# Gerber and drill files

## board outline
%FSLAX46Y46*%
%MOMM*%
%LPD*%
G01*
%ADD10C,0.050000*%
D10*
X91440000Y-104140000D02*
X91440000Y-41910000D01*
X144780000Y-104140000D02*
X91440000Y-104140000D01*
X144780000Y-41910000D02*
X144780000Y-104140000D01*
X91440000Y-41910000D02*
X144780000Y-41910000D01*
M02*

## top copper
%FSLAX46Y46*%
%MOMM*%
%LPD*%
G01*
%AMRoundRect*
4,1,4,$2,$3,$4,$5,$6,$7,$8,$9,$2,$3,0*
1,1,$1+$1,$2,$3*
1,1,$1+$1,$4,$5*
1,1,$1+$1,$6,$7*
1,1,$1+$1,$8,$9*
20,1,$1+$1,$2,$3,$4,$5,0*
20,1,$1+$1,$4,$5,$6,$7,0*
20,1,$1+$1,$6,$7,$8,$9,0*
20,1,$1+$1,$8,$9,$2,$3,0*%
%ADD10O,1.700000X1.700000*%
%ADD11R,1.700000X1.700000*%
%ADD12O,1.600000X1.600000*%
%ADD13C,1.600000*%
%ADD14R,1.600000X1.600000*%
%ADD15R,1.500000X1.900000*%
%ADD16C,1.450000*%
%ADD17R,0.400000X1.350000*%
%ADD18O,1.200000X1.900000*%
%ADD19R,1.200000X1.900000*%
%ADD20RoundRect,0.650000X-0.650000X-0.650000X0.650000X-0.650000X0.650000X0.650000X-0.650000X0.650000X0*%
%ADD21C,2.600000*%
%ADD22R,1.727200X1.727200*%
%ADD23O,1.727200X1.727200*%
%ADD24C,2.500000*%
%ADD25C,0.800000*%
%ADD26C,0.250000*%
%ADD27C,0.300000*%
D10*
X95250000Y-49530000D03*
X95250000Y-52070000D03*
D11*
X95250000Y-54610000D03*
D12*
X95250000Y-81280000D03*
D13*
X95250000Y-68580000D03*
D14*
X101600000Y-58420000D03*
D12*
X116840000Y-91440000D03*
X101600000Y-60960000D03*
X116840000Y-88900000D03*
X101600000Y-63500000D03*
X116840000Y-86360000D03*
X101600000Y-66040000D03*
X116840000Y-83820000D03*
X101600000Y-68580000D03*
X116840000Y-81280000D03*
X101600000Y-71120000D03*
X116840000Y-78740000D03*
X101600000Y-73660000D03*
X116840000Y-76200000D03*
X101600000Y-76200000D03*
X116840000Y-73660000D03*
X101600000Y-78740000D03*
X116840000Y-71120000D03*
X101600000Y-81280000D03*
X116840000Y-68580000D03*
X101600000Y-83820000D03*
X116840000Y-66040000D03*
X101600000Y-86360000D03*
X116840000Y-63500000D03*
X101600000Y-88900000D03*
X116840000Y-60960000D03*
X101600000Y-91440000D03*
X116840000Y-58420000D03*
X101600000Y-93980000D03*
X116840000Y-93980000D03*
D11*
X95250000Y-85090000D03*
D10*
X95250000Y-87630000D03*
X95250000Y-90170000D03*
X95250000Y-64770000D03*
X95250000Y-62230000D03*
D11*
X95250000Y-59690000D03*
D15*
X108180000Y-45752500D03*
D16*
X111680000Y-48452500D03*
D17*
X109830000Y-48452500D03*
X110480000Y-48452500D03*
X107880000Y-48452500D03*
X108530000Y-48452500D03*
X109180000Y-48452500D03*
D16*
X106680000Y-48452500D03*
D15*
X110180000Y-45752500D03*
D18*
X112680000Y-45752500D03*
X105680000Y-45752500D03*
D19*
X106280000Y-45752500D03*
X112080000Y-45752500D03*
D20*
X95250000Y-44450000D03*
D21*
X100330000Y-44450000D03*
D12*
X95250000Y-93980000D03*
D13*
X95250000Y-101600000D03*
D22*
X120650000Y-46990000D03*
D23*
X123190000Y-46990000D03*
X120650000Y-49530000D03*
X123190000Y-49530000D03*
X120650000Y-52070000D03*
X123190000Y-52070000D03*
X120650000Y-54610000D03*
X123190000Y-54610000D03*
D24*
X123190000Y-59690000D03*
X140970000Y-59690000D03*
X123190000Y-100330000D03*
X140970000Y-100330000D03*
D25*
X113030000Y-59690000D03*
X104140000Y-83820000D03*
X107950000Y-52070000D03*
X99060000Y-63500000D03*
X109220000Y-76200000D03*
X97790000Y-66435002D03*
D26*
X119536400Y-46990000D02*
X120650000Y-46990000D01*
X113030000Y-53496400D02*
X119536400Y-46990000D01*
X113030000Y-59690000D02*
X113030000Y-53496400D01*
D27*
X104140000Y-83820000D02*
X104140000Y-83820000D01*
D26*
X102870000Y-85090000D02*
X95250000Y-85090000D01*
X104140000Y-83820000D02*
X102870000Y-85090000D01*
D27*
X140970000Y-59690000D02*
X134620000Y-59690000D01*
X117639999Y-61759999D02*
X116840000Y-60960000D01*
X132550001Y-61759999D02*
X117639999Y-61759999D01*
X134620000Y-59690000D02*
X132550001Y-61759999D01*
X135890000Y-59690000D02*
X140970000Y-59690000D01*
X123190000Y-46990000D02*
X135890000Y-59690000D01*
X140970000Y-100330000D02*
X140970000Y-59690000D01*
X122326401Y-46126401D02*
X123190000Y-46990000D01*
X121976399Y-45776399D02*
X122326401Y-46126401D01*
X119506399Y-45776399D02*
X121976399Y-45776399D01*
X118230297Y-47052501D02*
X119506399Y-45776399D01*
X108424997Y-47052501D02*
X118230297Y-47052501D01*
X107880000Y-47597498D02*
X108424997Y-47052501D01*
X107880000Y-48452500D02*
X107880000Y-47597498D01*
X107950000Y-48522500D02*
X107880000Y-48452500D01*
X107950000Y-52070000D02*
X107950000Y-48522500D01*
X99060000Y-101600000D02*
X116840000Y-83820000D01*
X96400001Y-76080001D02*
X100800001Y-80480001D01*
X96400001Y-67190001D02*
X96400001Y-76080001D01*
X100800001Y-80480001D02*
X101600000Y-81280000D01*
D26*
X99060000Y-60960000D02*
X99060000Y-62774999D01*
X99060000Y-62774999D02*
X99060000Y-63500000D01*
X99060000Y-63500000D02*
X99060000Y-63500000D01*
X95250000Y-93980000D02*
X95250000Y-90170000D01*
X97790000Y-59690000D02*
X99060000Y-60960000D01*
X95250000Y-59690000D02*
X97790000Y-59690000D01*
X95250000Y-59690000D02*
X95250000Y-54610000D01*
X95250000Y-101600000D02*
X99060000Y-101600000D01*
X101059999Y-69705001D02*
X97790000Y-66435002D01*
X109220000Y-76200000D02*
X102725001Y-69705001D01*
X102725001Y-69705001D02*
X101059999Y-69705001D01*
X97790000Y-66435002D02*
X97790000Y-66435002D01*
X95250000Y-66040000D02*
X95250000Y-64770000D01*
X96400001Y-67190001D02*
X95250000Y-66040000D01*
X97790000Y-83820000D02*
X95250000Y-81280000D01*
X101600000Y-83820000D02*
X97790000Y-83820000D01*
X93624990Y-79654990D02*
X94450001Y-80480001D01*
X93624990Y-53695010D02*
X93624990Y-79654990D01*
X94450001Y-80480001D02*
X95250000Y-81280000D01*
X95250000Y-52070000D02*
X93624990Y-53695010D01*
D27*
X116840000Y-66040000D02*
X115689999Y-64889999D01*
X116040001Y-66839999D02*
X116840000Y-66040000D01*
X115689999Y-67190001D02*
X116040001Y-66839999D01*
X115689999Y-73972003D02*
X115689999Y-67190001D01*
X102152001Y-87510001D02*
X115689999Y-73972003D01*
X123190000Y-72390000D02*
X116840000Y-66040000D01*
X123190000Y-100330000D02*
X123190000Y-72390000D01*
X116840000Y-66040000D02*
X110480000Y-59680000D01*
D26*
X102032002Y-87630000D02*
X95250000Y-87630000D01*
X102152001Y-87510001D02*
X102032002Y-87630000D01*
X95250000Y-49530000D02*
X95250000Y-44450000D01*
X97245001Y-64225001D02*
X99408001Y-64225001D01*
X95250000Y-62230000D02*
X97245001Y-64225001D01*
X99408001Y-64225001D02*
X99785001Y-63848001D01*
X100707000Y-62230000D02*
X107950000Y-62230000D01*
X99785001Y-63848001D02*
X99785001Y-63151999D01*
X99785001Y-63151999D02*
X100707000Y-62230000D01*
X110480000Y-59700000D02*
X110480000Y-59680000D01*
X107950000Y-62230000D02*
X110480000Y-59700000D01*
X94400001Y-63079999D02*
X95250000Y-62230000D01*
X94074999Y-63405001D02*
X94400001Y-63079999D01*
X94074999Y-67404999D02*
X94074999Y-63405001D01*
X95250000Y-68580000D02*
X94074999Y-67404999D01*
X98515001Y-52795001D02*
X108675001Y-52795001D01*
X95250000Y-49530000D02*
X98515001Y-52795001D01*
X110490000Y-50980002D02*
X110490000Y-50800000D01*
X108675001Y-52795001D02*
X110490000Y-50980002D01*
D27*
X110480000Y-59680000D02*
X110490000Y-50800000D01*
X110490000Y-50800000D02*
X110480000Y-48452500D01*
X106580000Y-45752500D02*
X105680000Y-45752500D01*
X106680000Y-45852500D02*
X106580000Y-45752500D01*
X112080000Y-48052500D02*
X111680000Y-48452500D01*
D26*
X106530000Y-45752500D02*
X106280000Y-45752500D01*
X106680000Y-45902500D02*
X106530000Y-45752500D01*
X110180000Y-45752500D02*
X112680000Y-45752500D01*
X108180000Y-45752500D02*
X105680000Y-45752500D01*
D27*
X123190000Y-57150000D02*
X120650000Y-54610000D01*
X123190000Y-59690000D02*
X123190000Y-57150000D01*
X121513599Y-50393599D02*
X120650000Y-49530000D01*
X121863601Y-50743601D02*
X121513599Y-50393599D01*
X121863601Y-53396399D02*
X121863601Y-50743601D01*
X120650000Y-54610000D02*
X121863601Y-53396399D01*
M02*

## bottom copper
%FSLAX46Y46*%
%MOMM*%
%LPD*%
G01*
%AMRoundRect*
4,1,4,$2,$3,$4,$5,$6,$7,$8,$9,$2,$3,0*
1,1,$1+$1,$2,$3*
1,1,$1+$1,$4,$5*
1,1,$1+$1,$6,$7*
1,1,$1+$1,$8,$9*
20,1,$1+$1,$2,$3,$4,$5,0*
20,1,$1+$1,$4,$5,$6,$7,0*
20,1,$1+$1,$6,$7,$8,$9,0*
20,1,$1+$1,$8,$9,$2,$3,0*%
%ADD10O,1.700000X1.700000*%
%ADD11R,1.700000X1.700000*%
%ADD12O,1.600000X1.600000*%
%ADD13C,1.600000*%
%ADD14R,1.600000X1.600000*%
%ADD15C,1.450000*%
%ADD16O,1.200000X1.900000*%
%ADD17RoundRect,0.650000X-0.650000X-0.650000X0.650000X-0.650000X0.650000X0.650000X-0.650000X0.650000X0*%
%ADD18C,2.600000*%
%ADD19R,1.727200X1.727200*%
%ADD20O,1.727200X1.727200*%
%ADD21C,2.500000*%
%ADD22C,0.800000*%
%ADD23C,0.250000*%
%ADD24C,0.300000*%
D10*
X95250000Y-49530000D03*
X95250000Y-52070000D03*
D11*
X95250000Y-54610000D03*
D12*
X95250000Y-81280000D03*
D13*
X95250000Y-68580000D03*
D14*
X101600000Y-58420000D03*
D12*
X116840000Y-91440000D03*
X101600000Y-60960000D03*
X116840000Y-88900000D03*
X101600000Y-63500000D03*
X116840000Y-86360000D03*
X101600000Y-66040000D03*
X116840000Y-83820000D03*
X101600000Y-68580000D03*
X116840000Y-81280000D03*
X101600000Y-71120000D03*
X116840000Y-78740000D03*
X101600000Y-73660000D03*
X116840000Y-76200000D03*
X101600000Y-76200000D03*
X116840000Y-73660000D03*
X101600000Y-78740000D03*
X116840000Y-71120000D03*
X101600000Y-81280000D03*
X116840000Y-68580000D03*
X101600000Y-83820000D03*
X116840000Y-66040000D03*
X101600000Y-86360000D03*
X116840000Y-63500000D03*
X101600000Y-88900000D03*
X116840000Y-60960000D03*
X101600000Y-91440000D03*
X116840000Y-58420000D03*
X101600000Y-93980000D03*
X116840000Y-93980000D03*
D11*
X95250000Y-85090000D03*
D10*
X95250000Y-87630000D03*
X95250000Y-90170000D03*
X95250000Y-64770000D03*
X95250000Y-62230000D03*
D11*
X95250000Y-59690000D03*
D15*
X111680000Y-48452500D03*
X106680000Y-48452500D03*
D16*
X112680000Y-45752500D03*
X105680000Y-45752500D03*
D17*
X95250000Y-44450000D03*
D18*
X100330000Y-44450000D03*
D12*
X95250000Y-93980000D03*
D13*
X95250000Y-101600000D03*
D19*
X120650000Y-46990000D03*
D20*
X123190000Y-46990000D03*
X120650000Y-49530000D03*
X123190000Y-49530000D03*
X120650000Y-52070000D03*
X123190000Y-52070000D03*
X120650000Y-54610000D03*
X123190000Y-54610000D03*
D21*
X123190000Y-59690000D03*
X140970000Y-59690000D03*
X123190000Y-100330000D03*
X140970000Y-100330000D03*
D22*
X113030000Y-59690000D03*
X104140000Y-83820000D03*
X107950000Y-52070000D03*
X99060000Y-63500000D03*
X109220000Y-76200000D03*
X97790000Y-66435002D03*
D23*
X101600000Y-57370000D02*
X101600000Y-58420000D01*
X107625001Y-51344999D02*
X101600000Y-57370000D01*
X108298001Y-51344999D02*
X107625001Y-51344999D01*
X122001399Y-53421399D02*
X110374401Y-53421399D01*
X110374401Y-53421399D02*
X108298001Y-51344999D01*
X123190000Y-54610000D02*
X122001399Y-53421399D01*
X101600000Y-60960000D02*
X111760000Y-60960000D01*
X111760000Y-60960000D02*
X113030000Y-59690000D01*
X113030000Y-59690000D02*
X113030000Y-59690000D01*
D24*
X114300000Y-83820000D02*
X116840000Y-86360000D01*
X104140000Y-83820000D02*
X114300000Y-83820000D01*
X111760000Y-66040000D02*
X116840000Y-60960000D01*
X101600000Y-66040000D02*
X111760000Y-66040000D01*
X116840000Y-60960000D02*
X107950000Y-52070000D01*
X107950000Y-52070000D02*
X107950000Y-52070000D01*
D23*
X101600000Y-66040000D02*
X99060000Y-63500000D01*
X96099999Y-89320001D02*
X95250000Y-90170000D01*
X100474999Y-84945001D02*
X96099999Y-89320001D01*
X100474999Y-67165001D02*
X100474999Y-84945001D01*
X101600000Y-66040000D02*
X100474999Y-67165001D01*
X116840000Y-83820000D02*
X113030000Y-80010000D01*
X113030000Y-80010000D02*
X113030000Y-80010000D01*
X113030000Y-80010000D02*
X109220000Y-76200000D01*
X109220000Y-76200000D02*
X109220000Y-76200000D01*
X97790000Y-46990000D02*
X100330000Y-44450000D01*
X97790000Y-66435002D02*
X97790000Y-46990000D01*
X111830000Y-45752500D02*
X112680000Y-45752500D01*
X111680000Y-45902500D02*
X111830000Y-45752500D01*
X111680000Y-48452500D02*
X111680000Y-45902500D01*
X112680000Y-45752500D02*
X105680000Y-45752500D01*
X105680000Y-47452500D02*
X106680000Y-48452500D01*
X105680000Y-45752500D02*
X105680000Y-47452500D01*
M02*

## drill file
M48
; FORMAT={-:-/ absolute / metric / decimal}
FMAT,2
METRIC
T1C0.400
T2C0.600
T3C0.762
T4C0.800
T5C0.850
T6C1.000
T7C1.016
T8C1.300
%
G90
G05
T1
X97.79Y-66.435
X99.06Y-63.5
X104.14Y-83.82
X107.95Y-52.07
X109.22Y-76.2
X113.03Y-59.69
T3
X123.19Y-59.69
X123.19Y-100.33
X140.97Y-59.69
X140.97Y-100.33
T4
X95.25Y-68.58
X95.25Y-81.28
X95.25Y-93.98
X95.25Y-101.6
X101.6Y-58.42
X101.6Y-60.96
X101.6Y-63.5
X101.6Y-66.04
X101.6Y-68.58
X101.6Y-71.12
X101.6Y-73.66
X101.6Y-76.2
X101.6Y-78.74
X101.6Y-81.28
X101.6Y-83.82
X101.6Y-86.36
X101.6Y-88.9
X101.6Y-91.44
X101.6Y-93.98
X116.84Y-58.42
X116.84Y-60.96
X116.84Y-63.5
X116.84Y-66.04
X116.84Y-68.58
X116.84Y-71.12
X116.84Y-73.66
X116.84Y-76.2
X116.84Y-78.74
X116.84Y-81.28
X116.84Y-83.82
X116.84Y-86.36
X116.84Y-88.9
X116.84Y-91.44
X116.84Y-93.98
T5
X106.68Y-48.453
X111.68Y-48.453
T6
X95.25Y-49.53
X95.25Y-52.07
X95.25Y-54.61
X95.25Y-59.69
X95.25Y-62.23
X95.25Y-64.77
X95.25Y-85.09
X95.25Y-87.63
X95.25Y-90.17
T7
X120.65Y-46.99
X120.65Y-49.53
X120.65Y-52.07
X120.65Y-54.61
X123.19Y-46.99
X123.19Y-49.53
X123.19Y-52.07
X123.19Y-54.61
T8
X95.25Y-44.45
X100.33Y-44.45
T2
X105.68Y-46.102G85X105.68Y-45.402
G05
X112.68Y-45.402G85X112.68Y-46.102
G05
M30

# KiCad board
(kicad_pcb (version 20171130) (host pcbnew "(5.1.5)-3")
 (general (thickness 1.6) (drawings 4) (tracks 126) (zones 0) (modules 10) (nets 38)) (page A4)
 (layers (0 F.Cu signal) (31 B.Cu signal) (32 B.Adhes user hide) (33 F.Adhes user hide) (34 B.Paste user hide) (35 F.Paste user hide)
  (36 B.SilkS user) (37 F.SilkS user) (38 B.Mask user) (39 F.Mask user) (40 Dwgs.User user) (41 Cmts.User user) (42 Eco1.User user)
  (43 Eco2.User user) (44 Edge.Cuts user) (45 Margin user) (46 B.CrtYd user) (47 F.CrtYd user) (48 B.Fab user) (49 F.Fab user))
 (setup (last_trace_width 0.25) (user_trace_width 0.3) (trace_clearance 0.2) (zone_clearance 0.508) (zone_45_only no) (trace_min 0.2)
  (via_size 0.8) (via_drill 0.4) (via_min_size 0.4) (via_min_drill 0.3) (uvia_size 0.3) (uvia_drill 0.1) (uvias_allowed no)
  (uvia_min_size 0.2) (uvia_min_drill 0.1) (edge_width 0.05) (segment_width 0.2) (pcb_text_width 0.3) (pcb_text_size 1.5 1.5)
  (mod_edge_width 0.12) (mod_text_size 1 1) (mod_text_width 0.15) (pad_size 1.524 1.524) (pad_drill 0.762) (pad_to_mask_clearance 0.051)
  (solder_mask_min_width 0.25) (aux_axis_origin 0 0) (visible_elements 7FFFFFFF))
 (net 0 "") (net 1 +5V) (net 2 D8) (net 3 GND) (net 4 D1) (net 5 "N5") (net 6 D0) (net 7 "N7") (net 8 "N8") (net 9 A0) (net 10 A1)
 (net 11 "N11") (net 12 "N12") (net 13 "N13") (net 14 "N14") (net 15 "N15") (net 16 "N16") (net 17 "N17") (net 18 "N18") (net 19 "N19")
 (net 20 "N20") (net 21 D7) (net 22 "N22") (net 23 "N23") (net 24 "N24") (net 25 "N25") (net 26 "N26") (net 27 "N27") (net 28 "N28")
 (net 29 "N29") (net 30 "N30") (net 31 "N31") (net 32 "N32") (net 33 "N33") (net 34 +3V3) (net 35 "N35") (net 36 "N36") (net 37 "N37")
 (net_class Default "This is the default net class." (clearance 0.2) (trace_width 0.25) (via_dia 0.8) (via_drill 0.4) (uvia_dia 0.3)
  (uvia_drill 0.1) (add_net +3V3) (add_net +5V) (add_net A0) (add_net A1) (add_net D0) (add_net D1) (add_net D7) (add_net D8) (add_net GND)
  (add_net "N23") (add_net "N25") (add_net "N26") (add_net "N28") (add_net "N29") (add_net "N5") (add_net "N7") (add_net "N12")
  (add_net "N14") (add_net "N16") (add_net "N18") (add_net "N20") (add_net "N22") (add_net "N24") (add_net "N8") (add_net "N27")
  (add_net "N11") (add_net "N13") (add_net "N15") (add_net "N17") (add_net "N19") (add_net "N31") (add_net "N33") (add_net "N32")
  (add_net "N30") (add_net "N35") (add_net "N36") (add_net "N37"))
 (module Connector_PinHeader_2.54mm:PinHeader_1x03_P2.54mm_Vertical (layer F.Cu) (at 95.25 54.61 180)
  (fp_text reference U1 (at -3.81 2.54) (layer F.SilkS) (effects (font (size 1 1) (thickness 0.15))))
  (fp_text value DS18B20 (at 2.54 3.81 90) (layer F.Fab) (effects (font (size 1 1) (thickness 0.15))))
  (pad 3 thru_hole oval (at 0 5.08 180) (size 1.7 1.7) (drill 1) (layers *.Cu *.Mask) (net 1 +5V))
  (pad 2 thru_hole oval (at 0 2.54 180) (size 1.7 1.7) (drill 1) (layers *.Cu *.Mask) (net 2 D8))
  (pad 1 thru_hole rect (at 0 0 180) (size 1.7 1.7) (drill 1) (layers *.Cu *.Mask) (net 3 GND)))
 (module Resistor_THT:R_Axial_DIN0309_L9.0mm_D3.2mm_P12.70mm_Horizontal (layer F.Cu) (at 95.25 68.58 270)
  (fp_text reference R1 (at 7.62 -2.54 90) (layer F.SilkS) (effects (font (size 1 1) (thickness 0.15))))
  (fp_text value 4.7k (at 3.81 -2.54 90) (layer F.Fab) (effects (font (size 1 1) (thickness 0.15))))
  (pad 2 thru_hole oval (at 12.7 0 270) (size 1.6 1.6) (drill 0.8) (layers *.Cu *.Mask) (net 2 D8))
  (pad 1 thru_hole circle (at 0 0 270) (size 1.6 1.6) (drill 0.8) (layers *.Cu *.Mask) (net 1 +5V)))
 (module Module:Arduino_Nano (layer F.Cu) (at 101.6 58.42)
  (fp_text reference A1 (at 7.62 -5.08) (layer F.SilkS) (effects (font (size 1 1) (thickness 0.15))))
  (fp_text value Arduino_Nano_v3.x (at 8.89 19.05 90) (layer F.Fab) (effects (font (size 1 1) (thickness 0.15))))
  (pad 1 thru_hole rect (at 0 0) (size 1.6 1.6) (drill 0.8) (layers *.Cu *.Mask) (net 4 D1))
  (pad 17 thru_hole oval (at 15.24 33.02) (size 1.6 1.6) (drill 0.8) (layers *.Cu *.Mask) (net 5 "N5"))
  (pad 2 thru_hole oval (at 0 2.54) (size 1.6 1.6) (drill 0.8) (layers *.Cu *.Mask) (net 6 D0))
  (pad 18 thru_hole oval (at 15.24 30.48) (size 1.6 1.6) (drill 0.8) (layers *.Cu *.Mask) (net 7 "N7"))
  (pad 3 thru_hole oval (at 0 5.08) (size 1.6 1.6) (drill 0.8) (layers *.Cu *.Mask) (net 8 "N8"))
  (pad 19 thru_hole oval (at 15.24 27.94) (size 1.6 1.6) (drill 0.8) (layers *.Cu *.Mask) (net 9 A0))
  (pad 4 thru_hole oval (at 0 7.62) (size 1.6 1.6) (drill 0.8) (layers *.Cu *.Mask) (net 3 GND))
  (pad 20 thru_hole oval (at 15.24 25.4) (size 1.6 1.6) (drill 0.8) (layers *.Cu *.Mask) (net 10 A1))
  (pad 5 thru_hole oval (at 0 10.16) (size 1.6 1.6) (drill 0.8) (layers *.Cu *.Mask) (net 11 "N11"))
  (pad 21 thru_hole oval (at 15.24 22.86) (size 1.6 1.6) (drill 0.8) (layers *.Cu *.Mask) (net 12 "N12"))
  (pad 6 thru_hole oval (at 0 12.7) (size 1.6 1.6) (drill 0.8) (layers *.Cu *.Mask) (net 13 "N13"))
  (pad 22 thru_hole oval (at 15.24 20.32) (size 1.6 1.6) (drill 0.8) (layers *.Cu *.Mask) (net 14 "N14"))
  (pad 7 thru_hole oval (at 0 15.24) (size 1.6 1.6) (drill 0.8) (layers *.Cu *.Mask) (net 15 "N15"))
  (pad 23 thru_hole oval (at 15.24 17.78) (size 1.6 1.6) (drill 0.8) (layers *.Cu *.Mask) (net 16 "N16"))
  (pad 8 thru_hole oval (at 0 17.78) (size 1.6 1.6) (drill 0.8) (layers *.Cu *.Mask) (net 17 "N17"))
  (pad 24 thru_hole oval (at 15.24 15.24) (size 1.6 1.6) (drill 0.8) (layers *.Cu *.Mask) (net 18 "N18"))
  (pad 9 thru_hole oval (at 0 20.32) (size 1.6 1.6) (drill 0.8) (layers *.Cu *.Mask) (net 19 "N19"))
  (pad 25 thru_hole oval (at 15.24 12.7) (size 1.6 1.6) (drill 0.8) (layers *.Cu *.Mask) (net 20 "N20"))
  (pad 10 thru_hole oval (at 0 22.86) (size 1.6 1.6) (drill 0.8) (layers *.Cu *.Mask) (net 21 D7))
  (pad 26 thru_hole oval (at 15.24 10.16) (size 1.6 1.6) (drill 0.8) (layers *.Cu *.Mask) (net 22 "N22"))
  (pad 11 thru_hole oval (at 0 25.4) (size 1.6 1.6) (drill 0.8) (layers *.Cu *.Mask) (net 2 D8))
  (pad 27 thru_hole oval (at 15.24 7.62) (size 1.6 1.6) (drill 0.8) (layers *.Cu *.Mask) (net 1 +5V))
  (pad 12 thru_hole oval (at 0 27.94) (size 1.6 1.6) (drill 0.8) (layers *.Cu *.Mask) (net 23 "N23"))
  (pad 28 thru_hole oval (at 15.24 5.08) (size 1.6 1.6) (drill 0.8) (layers *.Cu *.Mask) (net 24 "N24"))
  (pad 13 thru_hole oval (at 0 30.48) (size 1.6 1.6) (drill 0.8) (layers *.Cu *.Mask) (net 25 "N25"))
  (pad 29 thru_hole oval (at 15.24 2.54) (size 1.6 1.6) (drill 0.8) (layers *.Cu *.Mask) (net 3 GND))
  (pad 14 thru_hole oval (at 0 33.02) (size 1.6 1.6) (drill 0.8) (layers *.Cu *.Mask) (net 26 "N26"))
  (pad 30 thru_hole oval (at 15.24 0) (size 1.6 1.6) (drill 0.8) (layers *.Cu *.Mask) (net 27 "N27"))
  (pad 15 thru_hole oval (at 0 35.56) (size 1.6 1.6) (drill 0.8) (layers *.Cu *.Mask) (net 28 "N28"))
  (pad 16 thru_hole oval (at 15.24 35.56) (size 1.6 1.6) (drill 0.8) (layers *.Cu *.Mask) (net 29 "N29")))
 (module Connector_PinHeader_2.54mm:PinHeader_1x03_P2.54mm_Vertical (layer F.Cu) (at 95.25 85.09)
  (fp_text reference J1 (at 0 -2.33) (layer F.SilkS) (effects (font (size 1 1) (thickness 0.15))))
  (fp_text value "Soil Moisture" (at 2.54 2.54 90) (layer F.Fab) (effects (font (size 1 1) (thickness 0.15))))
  (pad 1 thru_hole rect (at 0 0) (size 1.7 1.7) (drill 1) (layers *.Cu *.Mask) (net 9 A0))
  (pad 2 thru_hole oval (at 0 2.54) (size 1.7 1.7) (drill 1) (layers *.Cu *.Mask) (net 1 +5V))
  (pad 3 thru_hole oval (at 0 5.08) (size 1.7 1.7) (drill 1) (layers *.Cu *.Mask) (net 3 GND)))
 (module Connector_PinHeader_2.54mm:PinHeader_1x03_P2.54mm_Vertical (layer F.Cu) (at 95.25 59.69)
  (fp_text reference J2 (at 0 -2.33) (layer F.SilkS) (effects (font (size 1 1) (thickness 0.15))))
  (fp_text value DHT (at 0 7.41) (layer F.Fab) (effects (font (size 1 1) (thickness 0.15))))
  (pad 3 thru_hole oval (at 0 5.08) (size 1.7 1.7) (drill 1) (layers *.Cu *.Mask) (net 21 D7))
  (pad 2 thru_hole oval (at 0 2.54) (size 1.7 1.7) (drill 1) (layers *.Cu *.Mask) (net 1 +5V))
  (pad 1 thru_hole rect (at 0 0) (size 1.7 1.7) (drill 1) (layers *.Cu *.Mask) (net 3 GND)))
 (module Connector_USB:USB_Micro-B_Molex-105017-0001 (layer F.Cu) (at 109.18 46.99 180)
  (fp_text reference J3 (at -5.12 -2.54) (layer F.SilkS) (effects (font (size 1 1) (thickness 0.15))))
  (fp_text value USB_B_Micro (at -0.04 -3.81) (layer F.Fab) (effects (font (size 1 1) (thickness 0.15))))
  (pad 6 smd rect (at 1 1.2375 180) (size 1.5 1.9) (layers F.Cu F.Paste F.Mask) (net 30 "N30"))
  (pad 6 thru_hole circle (at -2.5 -1.4625 180) (size 1.45 1.45) (drill 0.85) (layers *.Cu *.Mask) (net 30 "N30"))
  (pad 2 smd rect (at -0.65 -1.4625 180) (size 0.4 1.35) (layers F.Cu F.Paste F.Mask) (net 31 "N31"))
  (pad 1 smd rect (at -1.3 -1.4625 180) (size 0.4 1.35) (layers F.Cu F.Paste F.Mask) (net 1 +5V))
  (pad 5 smd rect (at 1.3 -1.4625 180) (size 0.4 1.35) (layers F.Cu F.Paste F.Mask) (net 3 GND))
  (pad 4 smd rect (at 0.65 -1.4625 180) (size 0.4 1.35) (layers F.Cu F.Paste F.Mask) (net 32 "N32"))
  (pad 3 smd rect (at 0 -1.4625 180) (size 0.4 1.35) (layers F.Cu F.Paste F.Mask) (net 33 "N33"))
  (pad 6 thru_hole circle (at 2.5 -1.4625 180) (size 1.45 1.45) (drill 0.85) (layers *.Cu *.Mask) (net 30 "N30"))
  (pad 6 smd rect (at -1 1.2375 180) (size 1.5 1.9) (layers F.Cu F.Paste F.Mask) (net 30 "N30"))
  (pad 6 thru_hole oval (at -3.5 1.2375) (size 1.2 1.9) (drill oval 0.6 1.3) (layers *.Cu *.Mask) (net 30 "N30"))
  (pad 6 thru_hole oval (at 3.5 1.2375 180) (size 1.2 1.9) (drill oval 0.6 1.3) (layers *.Cu *.Mask) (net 30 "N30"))
  (pad 6 smd rect (at 2.9 1.2375 180) (size 1.2 1.9) (layers F.Cu F.Mask) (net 30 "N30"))
  (pad 6 smd rect (at -2.9 1.2375 180) (size 1.2 1.9) (layers F.Cu F.Mask) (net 30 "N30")))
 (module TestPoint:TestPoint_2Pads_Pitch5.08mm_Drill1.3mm (layer F.Cu) (at 95.25 44.45)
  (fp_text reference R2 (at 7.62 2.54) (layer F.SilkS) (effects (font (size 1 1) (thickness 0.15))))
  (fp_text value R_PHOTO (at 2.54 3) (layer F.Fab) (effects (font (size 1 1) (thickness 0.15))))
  (pad 1 thru_hole roundrect (at 0 0) (size 2.6 2.6) (drill 1.3) (layers *.Cu *.Mask) (roundrect_rratio 0.25) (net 1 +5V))
  (pad 2 thru_hole circle (at 5.08 0) (size 2.6 2.6) (drill 1.3) (layers *.Cu *.Mask) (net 10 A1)))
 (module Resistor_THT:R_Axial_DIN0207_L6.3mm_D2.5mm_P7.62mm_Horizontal (layer F.Cu) (at 95.25 101.6 90)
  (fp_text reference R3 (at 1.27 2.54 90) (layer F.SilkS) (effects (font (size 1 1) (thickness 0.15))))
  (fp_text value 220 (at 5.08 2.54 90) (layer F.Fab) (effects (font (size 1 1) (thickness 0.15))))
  (pad 2 thru_hole oval (at 7.62 0 90) (size 1.6 1.6) (drill 0.8) (layers *.Cu *.Mask) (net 3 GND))
  (pad 1 thru_hole circle (at 0 0 90) (size 1.6 1.6) (drill 0.8) (layers *.Cu *.Mask) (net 10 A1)))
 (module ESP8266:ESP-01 (layer F.Cu) (at 120.65 46.99)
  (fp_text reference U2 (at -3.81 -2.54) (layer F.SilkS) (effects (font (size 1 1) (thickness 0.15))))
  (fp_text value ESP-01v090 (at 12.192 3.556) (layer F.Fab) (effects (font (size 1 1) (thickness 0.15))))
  (pad 1 thru_hole rect (at 0 0) (size 1.7272 1.7272) (drill 1.016) (layers *.Cu *.Mask F.SilkS) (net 6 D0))
  (pad 2 thru_hole oval (at 2.54 0) (size 1.7272 1.7272) (drill 1.016) (layers *.Cu *.Mask F.SilkS) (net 3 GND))
  (pad 3 thru_hole oval (at 0 2.54) (size 1.7272 1.7272) (drill 1.016) (layers *.Cu *.Mask F.SilkS) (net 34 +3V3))
  (pad 4 thru_hole oval (at 2.54 2.54) (size 1.7272 1.7272) (drill 1.016) (layers *.Cu *.Mask F.SilkS) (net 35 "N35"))
  (pad 5 thru_hole oval (at 0 5.08) (size 1.7272 1.7272) (drill 1.016) (layers *.Cu *.Mask F.SilkS) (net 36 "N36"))
  (pad 6 thru_hole oval (at 2.54 5.08) (size 1.7272 1.7272) (drill 1.016) (layers *.Cu *.Mask F.SilkS) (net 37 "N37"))
  (pad 7 thru_hole oval (at 0 7.62) (size 1.7272 1.7272) (drill 1.016) (layers *.Cu *.Mask F.SilkS) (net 34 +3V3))
  (pad 8 thru_hole oval (at 2.54 7.62) (size 1.7272 1.7272) (drill 1.016) (layers *.Cu *.Mask F.SilkS) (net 4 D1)))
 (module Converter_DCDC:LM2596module (layer F.Cu) (at 132.08 80.01)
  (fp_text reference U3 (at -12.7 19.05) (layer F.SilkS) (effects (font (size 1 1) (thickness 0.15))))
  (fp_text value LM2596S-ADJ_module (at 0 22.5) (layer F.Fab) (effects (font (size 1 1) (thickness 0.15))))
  (pad 4 thru_hole circle (at -8.89 -20.32) (size 2.5 2.5) (drill 0.762) (layers *.Cu *.Mask) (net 34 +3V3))
  (pad 3 thru_hole circle (at 8.89 -20.32) (size 2.5 2.5) (drill 0.762) (layers *.Cu *.Mask) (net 3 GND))
  (pad 1 thru_hole circle (at -8.89 20.32) (size 2.5 2.5) (drill 0.762) (layers *.Cu *.Mask) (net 1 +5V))
  (pad 2 thru_hole circle (at 8.89 20.32) (size 2.5 2.5) (drill 0.762) (layers *.Cu *.Mask) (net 3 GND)))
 (gr_line (start 91.44 104.14) (end 91.44 41.91) (layer Edge.Cuts) (width 0.05))
 (gr_line (start 144.78 104.14) (end 91.44 104.14) (layer Edge.Cuts) (width 0.05))
 (gr_line (start 144.78 41.91) (end 144.78 104.14) (layer Edge.Cuts) (width 0.05))
 (gr_line (start 91.44 41.91) (end 144.78 41.91) (layer Edge.Cuts) (width 0.05))
 (segment (start 101.6 57.37) (end 101.6 58.42) (width 0.25) (layer B.Cu) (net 4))
 (segment (start 107.625001 51.344999) (end 101.6 57.37) (width 0.25) (layer B.Cu) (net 4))
 (segment (start 108.298001 51.344999) (end 107.625001 51.344999) (width 0.25) (layer B.Cu) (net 4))
 (segment (start 122.001399 53.421399) (end 110.374401 53.421399) (width 0.25) (layer B.Cu) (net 4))
 (segment (start 110.374401 53.421399) (end 108.298001 51.344999) (width 0.25) (layer B.Cu) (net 4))
 (segment (start 123.19 54.61) (end 122.001399 53.421399) (width 0.25) (layer B.Cu) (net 4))
 (segment (start 101.6 60.96) (end 111.76 60.96) (width 0.25) (layer B.Cu) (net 6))
 (segment (start 111.76 60.96) (end 113.03 59.69) (width 0.25) (layer B.Cu) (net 6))
 (segment (start 113.03 59.69) (end 113.03 59.69) (width 0.25) (layer B.Cu) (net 6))
 (via (at 113.03 59.69) (size 0.8) (drill 0.4) (layers F.Cu B.Cu) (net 6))
 (segment (start 119.5364 46.99) (end 120.65 46.99) (width 0.25) (layer F.Cu) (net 6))
 (segment (start 113.03 53.4964) (end 119.5364 46.99) (width 0.25) (layer F.Cu) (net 6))
 (segment (start 113.03 59.69) (end 113.03 53.4964) (width 0.25) (layer F.Cu) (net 6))
 (segment (start 104.14 83.82) (end 104.14 83.82) (width 0.3) (layer F.Cu) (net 9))
 (via (at 104.14 83.82) (size 0.8) (drill 0.4) (layers F.Cu B.Cu) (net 9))
 (segment (start 114.3 83.82) (end 116.84 86.36) (width 0.3) (layer B.Cu) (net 9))
 (segment (start 104.14 83.82) (end 114.3 83.82) (width 0.3) (layer B.Cu) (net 9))
 (segment (start 102.87 85.09) (end 95.25 85.09) (width 0.25) (layer F.Cu) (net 9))
 (segment (start 104.14 83.82) (end 102.87 85.09) (width 0.25) (layer F.Cu) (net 9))
 (segment (start 111.76 66.04) (end 116.84 60.96) (width 0.3) (layer B.Cu) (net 3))
 (segment (start 101.6 66.04) (end 111.76 66.04) (width 0.3) (layer B.Cu) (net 3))
 (segment (start 140.97 59.69) (end 134.62 59.69) (width 0.3) (layer F.Cu) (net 3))
 (segment (start 117.639999 61.759999) (end 116.84 60.96) (width 0.3) (layer F.Cu) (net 3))
 (segment (start 132.550001 61.759999) (end 117.639999 61.759999) (width 0.3) (layer F.Cu) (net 3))
 (segment (start 134.62 59.69) (end 132.550001 61.759999) (width 0.3) (layer F.Cu) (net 3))
 (segment (start 135.89 59.69) (end 140.97 59.69) (width 0.3) (layer F.Cu) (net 3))
 (segment (start 123.19 46.99) (end 135.89 59.69) (width 0.3) (layer F.Cu) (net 3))
 (segment (start 140.97 100.33) (end 140.97 59.69) (width 0.3) (layer F.Cu) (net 3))
 (segment (start 122.326401 46.126401) (end 123.19 46.99) (width 0.3) (layer F.Cu) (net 3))
 (segment (start 121.976399 45.776399) (end 122.326401 46.126401) (width 0.3) (layer F.Cu) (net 3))
 (segment (start 119.506399 45.776399) (end 121.976399 45.776399) (width 0.3) (layer F.Cu) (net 3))
 (segment (start 118.230297 47.052501) (end 119.506399 45.776399) (width 0.3) (layer F.Cu) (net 3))
 (segment (start 108.424997 47.052501) (end 118.230297 47.052501) (width 0.3) (layer F.Cu) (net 3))
 (segment (start 107.88 47.597498) (end 108.424997 47.052501) (width 0.3) (layer F.Cu) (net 3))
 (segment (start 107.88 48.4525) (end 107.88 47.597498) (width 0.3) (layer F.Cu) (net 3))
 (segment (start 116.84 60.96) (end 107.95 52.07) (width 0.3) (layer B.Cu) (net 3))
 (segment (start 107.95 52.07) (end 107.95 52.07) (width 0.3) (layer B.Cu) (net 3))
 (via (at 107.95 52.07) (size 0.8) (drill 0.4) (layers F.Cu B.Cu) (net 3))
 (segment (start 107.95 48.5225) (end 107.88 48.4525) (width 0.3) (layer F.Cu) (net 3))
 (segment (start 107.95 52.07) (end 107.95 48.5225) (width 0.3) (layer F.Cu) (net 3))
 (segment (start 99.06 101.6) (end 116.84 83.82) (width 0.3) (layer F.Cu) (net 10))
 (segment (start 96.400001 76.080001) (end 100.800001 80.480001) (width 0.3) (layer F.Cu) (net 21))
 (segment (start 96.400001 67.190001) (end 96.400001 76.080001) (width 0.3) (layer F.Cu) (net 21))
 (segment (start 100.800001 80.480001) (end 101.6 81.28) (width 0.3) (layer F.Cu) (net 21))
 (segment (start 99.06 60.96) (end 99.06 62.774999) (width 0.25) (layer F.Cu) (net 3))
 (segment (start 99.06 62.774999) (end 99.06 63.5) (width 0.25) (layer F.Cu) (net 3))
 (segment (start 99.06 63.5) (end 99.06 63.5) (width 0.25) (layer F.Cu) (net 3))
 (via (at 99.06 63.5) (size 0.8) (drill 0.4) (layers F.Cu B.Cu) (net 3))
 (segment (start 95.25 93.98) (end 95.25 90.17) (width 0.25) (layer F.Cu) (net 3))
 (segment (start 97.79 59.69) (end 99.06 60.96) (width 0.25) (layer F.Cu) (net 3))
 (segment (start 95.25 59.69) (end 97.79 59.69) (width 0.25) (layer F.Cu) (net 3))
 (segment (start 95.25 59.69) (end 95.25 54.61) (width 0.25) (layer F.Cu) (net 3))
 (segment (start 101.6 66.04) (end 99.06 63.5) (width 0.25) (layer B.Cu) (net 3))
 (segment (start 96.099999 89.320001) (end 95.25 90.17) (width 0.25) (layer B.Cu) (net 3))
 (segment (start 100.474999 84.945001) (end 96.099999 89.320001) (width 0.25) (layer B.Cu) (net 3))
 (segment (start 100.474999 67.165001) (end 100.474999 84.945001) (width 0.25) (layer B.Cu) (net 3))
 (segment (start 101.6 66.04) (end 100.474999 67.165001) (width 0.25) (layer B.Cu) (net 3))
 (segment (start 95.25 101.6) (end 99.06 101.6) (width 0.25) (layer F.Cu) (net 10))
 (segment (start 116.84 83.82) (end 113.03 80.01) (width 0.25) (layer B.Cu) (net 10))
 (segment (start 113.03 80.01) (end 113.03 80.01) (width 0.25) (layer B.Cu) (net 10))
 (segment (start 113.03 80.01) (end 109.22 76.2) (width 0.25) (layer B.Cu) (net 10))
 (segment (start 109.22 76.2) (end 109.22 76.2) (width 0.25) (layer B.Cu) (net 10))
 (via (at 109.22 76.2) (size 0.8) (drill 0.4) (layers F.Cu B.Cu) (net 10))
 (segment (start 101.059999 69.705001) (end 97.79 66.435002) (width 0.25) (layer F.Cu) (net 10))
 (segment (start 109.22 76.2) (end 102.725001 69.705001) (width 0.25) (layer F.Cu) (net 10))
 (segment (start 102.725001 69.705001) (end 101.059999 69.705001) (width 0.25) (layer F.Cu) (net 10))
 (segment (start 97.79 66.435002) (end 97.79 66.435002) (width 0.25) (layer F.Cu) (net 10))
 (via (at 97.79 66.435002) (size 0.8) (drill 0.4) (layers F.Cu B.Cu) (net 10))
 (segment (start 97.79 46.99) (end 100.33 44.45) (width 0.25) (layer B.Cu) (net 10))
 (segment (start 97.79 66.435002) (end 97.79 46.99) (width 0.25) (layer B.Cu) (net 10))
 (segment (start 95.25 66.04) (end 95.25 64.77) (width 0.25) (layer F.Cu) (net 21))
 (segment (start 96.400001 67.190001) (end 95.25 66.04) (width 0.25) (layer F.Cu) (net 21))
 (segment (start 97.79 83.82) (end 95.25 81.28) (width 0.25) (layer F.Cu) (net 2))
 (segment (start 101.6 83.82) (end 97.79 83.82) (width 0.25) (layer F.Cu) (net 2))
 (segment (start 93.62499 79.65499) (end 94.450001 80.480001) (width 0.25) (layer F.Cu) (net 2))
 (segment (start 93.62499 53.69501) (end 93.62499 79.65499) (width 0.25) (layer F.Cu) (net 2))
 (segment (start 94.450001 80.480001) (end 95.25 81.28) (width 0.25) (layer F.Cu) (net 2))
 (segment (start 95.25 52.07) (end 93.62499 53.69501) (width 0.25) (layer F.Cu) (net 2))
 (segment (start 116.84 66.04) (end 115.689999 64.889999) (width 0.3) (layer F.Cu) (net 1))
 (segment (start 116.040001 66.839999) (end 116.84 66.04) (width 0.3) (layer F.Cu) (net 1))
 (segment (start 115.689999 67.190001) (end 116.040001 66.839999) (width 0.3) (layer F.Cu) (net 1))
 (segment (start 115.689999 73.972003) (end 115.689999 67.190001) (width 0.3) (layer F.Cu) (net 1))
 (segment (start 102.152001 87.510001) (end 115.689999 73.972003) (width 0.3) (layer F.Cu) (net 1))
 (segment (start 123.19 72.39) (end 116.84 66.04) (width 0.3) (layer F.Cu) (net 1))
 (segment (start 123.19 100.33) (end 123.19 72.39) (width 0.3) (layer F.Cu) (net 1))
 (segment (start 116.84 66.04) (end 110.48 59.68) (width 0.3) (layer F.Cu) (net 1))
 (segment (start 102.032002 87.63) (end 95.25 87.63) (width 0.25) (layer F.Cu) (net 1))
 (segment (start 102.152001 87.510001) (end 102.032002 87.63) (width 0.25) (layer F.Cu) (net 1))
 (segment (start 95.25 49.53) (end 95.25 44.45) (width 0.25) (layer F.Cu) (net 1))
 (segment (start 97.245001 64.225001) (end 99.408001 64.225001) (width 0.25) (layer F.Cu) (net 1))
 (segment (start 95.25 62.23) (end 97.245001 64.225001) (width 0.25) (layer F.Cu) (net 1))
 (segment (start 99.408001 64.225001) (end 99.785001 63.848001) (width 0.25) (layer F.Cu) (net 1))
 (segment (start 100.707 62.23) (end 107.95 62.23) (width 0.25) (layer F.Cu) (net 1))
 (segment (start 99.785001 63.848001) (end 99.785001 63.151999) (width 0.25) (layer F.Cu) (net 1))
 (segment (start 99.785001 63.151999) (end 100.707 62.23) (width 0.25) (layer F.Cu) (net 1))
 (segment (start 110.48 59.7) (end 110.48 59.68) (width 0.25) (layer F.Cu) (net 1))
 (segment (start 107.95 62.23) (end 110.48 59.7) (width 0.25) (layer F.Cu) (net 1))
 (segment (start 94.400001 63.079999) (end 95.25 62.23) (width 0.25) (layer F.Cu) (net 1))
 (segment (start 94.074999 63.405001) (end 94.400001 63.079999) (width 0.25) (layer F.Cu) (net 1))
 (segment (start 94.074999 67.404999) (end 94.074999 63.405001) (width 0.25) (layer F.Cu) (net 1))
 (segment (start 95.25 68.58) (end 94.074999 67.404999) (width 0.25) (layer F.Cu) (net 1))
 (segment (start 98.515001 52.795001) (end 108.675001 52.795001) (width 0.25) (layer F.Cu) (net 1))
 (segment (start 95.25 49.53) (end 98.515001 52.795001) (width 0.25) (layer F.Cu) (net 1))
 (segment (start 110.49 50.980002) (end 110.49 50.8) (width 0.25) (layer F.Cu) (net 1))
 (segment (start 108.675001 52.795001) (end 110.49 50.980002) (width 0.25) (layer F.Cu) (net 1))
 (segment (start 110.48 59.68) (end 110.49 50.8) (width 0.3) (layer F.Cu) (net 1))
 (segment (start 110.49 50.8) (end 110.48 48.4525) (width 0.3) (layer F.Cu) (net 1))
 (segment (start 106.58 45.7525) (end 105.68 45.7525) (width 0.3) (layer F.Cu) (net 30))
 (segment (start 106.68 45.8525) (end 106.58 45.7525) (width 0.3) (layer F.Cu) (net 30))
 (segment (start 112.08 48.0525) (end 111.68 48.4525) (width 0.3) (layer F.Cu) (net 30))
 (segment (start 106.53 45.7525) (end 106.28 45.7525) (width 0.25) (layer F.Cu) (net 30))
 (segment (start 106.68 45.9025) (end 106.53 45.7525) (width 0.25) (layer F.Cu) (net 30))
 (segment (start 111.83 45.7525) (end 112.68 45.7525) (width 0.25) (layer B.Cu) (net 30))
 (segment (start 111.68 45.9025) (end 111.83 45.7525) (width 0.25) (layer B.Cu) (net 30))
 (segment (start 111.68 48.4525) (end 111.68 45.9025) (width 0.25) (layer B.Cu) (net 30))
 (segment (start 112.68 45.7525) (end 105.68 45.7525) (width 0.25) (layer B.Cu) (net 30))
 (segment (start 105.68 47.4525) (end 106.68 48.4525) (width 0.25) (layer B.Cu) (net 30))
 (segment (start 105.68 45.7525) (end 105.68 47.4525) (width 0.25) (layer B.Cu) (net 30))
 (segment (start 110.18 45.7525) (end 112.68 45.7525) (width 0.25) (layer F.Cu) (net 30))
 (segment (start 108.18 45.7525) (end 105.68 45.7525) (width 0.25) (layer F.Cu) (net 30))
 (segment (start 123.19 57.15) (end 120.65 54.61) (width 0.3) (layer F.Cu) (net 34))
 (segment (start 123.19 59.69) (end 123.19 57.15) (width 0.3) (layer F.Cu) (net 34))
 (segment (start 121.513599 50.393599) (end 120.65 49.53) (width 0.3) (layer F.Cu) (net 34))
 (segment (start 121.863601 50.743601) (end 121.513599 50.393599) (width 0.3) (layer F.Cu) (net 34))
 (segment (start 121.863601 53.396399) (end 121.863601 50.743601) (width 0.3) (layer F.Cu) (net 34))
 (segment (start 120.65 54.61) (end 121.863601 53.396399) (width 0.3) (layer F.Cu) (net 34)))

